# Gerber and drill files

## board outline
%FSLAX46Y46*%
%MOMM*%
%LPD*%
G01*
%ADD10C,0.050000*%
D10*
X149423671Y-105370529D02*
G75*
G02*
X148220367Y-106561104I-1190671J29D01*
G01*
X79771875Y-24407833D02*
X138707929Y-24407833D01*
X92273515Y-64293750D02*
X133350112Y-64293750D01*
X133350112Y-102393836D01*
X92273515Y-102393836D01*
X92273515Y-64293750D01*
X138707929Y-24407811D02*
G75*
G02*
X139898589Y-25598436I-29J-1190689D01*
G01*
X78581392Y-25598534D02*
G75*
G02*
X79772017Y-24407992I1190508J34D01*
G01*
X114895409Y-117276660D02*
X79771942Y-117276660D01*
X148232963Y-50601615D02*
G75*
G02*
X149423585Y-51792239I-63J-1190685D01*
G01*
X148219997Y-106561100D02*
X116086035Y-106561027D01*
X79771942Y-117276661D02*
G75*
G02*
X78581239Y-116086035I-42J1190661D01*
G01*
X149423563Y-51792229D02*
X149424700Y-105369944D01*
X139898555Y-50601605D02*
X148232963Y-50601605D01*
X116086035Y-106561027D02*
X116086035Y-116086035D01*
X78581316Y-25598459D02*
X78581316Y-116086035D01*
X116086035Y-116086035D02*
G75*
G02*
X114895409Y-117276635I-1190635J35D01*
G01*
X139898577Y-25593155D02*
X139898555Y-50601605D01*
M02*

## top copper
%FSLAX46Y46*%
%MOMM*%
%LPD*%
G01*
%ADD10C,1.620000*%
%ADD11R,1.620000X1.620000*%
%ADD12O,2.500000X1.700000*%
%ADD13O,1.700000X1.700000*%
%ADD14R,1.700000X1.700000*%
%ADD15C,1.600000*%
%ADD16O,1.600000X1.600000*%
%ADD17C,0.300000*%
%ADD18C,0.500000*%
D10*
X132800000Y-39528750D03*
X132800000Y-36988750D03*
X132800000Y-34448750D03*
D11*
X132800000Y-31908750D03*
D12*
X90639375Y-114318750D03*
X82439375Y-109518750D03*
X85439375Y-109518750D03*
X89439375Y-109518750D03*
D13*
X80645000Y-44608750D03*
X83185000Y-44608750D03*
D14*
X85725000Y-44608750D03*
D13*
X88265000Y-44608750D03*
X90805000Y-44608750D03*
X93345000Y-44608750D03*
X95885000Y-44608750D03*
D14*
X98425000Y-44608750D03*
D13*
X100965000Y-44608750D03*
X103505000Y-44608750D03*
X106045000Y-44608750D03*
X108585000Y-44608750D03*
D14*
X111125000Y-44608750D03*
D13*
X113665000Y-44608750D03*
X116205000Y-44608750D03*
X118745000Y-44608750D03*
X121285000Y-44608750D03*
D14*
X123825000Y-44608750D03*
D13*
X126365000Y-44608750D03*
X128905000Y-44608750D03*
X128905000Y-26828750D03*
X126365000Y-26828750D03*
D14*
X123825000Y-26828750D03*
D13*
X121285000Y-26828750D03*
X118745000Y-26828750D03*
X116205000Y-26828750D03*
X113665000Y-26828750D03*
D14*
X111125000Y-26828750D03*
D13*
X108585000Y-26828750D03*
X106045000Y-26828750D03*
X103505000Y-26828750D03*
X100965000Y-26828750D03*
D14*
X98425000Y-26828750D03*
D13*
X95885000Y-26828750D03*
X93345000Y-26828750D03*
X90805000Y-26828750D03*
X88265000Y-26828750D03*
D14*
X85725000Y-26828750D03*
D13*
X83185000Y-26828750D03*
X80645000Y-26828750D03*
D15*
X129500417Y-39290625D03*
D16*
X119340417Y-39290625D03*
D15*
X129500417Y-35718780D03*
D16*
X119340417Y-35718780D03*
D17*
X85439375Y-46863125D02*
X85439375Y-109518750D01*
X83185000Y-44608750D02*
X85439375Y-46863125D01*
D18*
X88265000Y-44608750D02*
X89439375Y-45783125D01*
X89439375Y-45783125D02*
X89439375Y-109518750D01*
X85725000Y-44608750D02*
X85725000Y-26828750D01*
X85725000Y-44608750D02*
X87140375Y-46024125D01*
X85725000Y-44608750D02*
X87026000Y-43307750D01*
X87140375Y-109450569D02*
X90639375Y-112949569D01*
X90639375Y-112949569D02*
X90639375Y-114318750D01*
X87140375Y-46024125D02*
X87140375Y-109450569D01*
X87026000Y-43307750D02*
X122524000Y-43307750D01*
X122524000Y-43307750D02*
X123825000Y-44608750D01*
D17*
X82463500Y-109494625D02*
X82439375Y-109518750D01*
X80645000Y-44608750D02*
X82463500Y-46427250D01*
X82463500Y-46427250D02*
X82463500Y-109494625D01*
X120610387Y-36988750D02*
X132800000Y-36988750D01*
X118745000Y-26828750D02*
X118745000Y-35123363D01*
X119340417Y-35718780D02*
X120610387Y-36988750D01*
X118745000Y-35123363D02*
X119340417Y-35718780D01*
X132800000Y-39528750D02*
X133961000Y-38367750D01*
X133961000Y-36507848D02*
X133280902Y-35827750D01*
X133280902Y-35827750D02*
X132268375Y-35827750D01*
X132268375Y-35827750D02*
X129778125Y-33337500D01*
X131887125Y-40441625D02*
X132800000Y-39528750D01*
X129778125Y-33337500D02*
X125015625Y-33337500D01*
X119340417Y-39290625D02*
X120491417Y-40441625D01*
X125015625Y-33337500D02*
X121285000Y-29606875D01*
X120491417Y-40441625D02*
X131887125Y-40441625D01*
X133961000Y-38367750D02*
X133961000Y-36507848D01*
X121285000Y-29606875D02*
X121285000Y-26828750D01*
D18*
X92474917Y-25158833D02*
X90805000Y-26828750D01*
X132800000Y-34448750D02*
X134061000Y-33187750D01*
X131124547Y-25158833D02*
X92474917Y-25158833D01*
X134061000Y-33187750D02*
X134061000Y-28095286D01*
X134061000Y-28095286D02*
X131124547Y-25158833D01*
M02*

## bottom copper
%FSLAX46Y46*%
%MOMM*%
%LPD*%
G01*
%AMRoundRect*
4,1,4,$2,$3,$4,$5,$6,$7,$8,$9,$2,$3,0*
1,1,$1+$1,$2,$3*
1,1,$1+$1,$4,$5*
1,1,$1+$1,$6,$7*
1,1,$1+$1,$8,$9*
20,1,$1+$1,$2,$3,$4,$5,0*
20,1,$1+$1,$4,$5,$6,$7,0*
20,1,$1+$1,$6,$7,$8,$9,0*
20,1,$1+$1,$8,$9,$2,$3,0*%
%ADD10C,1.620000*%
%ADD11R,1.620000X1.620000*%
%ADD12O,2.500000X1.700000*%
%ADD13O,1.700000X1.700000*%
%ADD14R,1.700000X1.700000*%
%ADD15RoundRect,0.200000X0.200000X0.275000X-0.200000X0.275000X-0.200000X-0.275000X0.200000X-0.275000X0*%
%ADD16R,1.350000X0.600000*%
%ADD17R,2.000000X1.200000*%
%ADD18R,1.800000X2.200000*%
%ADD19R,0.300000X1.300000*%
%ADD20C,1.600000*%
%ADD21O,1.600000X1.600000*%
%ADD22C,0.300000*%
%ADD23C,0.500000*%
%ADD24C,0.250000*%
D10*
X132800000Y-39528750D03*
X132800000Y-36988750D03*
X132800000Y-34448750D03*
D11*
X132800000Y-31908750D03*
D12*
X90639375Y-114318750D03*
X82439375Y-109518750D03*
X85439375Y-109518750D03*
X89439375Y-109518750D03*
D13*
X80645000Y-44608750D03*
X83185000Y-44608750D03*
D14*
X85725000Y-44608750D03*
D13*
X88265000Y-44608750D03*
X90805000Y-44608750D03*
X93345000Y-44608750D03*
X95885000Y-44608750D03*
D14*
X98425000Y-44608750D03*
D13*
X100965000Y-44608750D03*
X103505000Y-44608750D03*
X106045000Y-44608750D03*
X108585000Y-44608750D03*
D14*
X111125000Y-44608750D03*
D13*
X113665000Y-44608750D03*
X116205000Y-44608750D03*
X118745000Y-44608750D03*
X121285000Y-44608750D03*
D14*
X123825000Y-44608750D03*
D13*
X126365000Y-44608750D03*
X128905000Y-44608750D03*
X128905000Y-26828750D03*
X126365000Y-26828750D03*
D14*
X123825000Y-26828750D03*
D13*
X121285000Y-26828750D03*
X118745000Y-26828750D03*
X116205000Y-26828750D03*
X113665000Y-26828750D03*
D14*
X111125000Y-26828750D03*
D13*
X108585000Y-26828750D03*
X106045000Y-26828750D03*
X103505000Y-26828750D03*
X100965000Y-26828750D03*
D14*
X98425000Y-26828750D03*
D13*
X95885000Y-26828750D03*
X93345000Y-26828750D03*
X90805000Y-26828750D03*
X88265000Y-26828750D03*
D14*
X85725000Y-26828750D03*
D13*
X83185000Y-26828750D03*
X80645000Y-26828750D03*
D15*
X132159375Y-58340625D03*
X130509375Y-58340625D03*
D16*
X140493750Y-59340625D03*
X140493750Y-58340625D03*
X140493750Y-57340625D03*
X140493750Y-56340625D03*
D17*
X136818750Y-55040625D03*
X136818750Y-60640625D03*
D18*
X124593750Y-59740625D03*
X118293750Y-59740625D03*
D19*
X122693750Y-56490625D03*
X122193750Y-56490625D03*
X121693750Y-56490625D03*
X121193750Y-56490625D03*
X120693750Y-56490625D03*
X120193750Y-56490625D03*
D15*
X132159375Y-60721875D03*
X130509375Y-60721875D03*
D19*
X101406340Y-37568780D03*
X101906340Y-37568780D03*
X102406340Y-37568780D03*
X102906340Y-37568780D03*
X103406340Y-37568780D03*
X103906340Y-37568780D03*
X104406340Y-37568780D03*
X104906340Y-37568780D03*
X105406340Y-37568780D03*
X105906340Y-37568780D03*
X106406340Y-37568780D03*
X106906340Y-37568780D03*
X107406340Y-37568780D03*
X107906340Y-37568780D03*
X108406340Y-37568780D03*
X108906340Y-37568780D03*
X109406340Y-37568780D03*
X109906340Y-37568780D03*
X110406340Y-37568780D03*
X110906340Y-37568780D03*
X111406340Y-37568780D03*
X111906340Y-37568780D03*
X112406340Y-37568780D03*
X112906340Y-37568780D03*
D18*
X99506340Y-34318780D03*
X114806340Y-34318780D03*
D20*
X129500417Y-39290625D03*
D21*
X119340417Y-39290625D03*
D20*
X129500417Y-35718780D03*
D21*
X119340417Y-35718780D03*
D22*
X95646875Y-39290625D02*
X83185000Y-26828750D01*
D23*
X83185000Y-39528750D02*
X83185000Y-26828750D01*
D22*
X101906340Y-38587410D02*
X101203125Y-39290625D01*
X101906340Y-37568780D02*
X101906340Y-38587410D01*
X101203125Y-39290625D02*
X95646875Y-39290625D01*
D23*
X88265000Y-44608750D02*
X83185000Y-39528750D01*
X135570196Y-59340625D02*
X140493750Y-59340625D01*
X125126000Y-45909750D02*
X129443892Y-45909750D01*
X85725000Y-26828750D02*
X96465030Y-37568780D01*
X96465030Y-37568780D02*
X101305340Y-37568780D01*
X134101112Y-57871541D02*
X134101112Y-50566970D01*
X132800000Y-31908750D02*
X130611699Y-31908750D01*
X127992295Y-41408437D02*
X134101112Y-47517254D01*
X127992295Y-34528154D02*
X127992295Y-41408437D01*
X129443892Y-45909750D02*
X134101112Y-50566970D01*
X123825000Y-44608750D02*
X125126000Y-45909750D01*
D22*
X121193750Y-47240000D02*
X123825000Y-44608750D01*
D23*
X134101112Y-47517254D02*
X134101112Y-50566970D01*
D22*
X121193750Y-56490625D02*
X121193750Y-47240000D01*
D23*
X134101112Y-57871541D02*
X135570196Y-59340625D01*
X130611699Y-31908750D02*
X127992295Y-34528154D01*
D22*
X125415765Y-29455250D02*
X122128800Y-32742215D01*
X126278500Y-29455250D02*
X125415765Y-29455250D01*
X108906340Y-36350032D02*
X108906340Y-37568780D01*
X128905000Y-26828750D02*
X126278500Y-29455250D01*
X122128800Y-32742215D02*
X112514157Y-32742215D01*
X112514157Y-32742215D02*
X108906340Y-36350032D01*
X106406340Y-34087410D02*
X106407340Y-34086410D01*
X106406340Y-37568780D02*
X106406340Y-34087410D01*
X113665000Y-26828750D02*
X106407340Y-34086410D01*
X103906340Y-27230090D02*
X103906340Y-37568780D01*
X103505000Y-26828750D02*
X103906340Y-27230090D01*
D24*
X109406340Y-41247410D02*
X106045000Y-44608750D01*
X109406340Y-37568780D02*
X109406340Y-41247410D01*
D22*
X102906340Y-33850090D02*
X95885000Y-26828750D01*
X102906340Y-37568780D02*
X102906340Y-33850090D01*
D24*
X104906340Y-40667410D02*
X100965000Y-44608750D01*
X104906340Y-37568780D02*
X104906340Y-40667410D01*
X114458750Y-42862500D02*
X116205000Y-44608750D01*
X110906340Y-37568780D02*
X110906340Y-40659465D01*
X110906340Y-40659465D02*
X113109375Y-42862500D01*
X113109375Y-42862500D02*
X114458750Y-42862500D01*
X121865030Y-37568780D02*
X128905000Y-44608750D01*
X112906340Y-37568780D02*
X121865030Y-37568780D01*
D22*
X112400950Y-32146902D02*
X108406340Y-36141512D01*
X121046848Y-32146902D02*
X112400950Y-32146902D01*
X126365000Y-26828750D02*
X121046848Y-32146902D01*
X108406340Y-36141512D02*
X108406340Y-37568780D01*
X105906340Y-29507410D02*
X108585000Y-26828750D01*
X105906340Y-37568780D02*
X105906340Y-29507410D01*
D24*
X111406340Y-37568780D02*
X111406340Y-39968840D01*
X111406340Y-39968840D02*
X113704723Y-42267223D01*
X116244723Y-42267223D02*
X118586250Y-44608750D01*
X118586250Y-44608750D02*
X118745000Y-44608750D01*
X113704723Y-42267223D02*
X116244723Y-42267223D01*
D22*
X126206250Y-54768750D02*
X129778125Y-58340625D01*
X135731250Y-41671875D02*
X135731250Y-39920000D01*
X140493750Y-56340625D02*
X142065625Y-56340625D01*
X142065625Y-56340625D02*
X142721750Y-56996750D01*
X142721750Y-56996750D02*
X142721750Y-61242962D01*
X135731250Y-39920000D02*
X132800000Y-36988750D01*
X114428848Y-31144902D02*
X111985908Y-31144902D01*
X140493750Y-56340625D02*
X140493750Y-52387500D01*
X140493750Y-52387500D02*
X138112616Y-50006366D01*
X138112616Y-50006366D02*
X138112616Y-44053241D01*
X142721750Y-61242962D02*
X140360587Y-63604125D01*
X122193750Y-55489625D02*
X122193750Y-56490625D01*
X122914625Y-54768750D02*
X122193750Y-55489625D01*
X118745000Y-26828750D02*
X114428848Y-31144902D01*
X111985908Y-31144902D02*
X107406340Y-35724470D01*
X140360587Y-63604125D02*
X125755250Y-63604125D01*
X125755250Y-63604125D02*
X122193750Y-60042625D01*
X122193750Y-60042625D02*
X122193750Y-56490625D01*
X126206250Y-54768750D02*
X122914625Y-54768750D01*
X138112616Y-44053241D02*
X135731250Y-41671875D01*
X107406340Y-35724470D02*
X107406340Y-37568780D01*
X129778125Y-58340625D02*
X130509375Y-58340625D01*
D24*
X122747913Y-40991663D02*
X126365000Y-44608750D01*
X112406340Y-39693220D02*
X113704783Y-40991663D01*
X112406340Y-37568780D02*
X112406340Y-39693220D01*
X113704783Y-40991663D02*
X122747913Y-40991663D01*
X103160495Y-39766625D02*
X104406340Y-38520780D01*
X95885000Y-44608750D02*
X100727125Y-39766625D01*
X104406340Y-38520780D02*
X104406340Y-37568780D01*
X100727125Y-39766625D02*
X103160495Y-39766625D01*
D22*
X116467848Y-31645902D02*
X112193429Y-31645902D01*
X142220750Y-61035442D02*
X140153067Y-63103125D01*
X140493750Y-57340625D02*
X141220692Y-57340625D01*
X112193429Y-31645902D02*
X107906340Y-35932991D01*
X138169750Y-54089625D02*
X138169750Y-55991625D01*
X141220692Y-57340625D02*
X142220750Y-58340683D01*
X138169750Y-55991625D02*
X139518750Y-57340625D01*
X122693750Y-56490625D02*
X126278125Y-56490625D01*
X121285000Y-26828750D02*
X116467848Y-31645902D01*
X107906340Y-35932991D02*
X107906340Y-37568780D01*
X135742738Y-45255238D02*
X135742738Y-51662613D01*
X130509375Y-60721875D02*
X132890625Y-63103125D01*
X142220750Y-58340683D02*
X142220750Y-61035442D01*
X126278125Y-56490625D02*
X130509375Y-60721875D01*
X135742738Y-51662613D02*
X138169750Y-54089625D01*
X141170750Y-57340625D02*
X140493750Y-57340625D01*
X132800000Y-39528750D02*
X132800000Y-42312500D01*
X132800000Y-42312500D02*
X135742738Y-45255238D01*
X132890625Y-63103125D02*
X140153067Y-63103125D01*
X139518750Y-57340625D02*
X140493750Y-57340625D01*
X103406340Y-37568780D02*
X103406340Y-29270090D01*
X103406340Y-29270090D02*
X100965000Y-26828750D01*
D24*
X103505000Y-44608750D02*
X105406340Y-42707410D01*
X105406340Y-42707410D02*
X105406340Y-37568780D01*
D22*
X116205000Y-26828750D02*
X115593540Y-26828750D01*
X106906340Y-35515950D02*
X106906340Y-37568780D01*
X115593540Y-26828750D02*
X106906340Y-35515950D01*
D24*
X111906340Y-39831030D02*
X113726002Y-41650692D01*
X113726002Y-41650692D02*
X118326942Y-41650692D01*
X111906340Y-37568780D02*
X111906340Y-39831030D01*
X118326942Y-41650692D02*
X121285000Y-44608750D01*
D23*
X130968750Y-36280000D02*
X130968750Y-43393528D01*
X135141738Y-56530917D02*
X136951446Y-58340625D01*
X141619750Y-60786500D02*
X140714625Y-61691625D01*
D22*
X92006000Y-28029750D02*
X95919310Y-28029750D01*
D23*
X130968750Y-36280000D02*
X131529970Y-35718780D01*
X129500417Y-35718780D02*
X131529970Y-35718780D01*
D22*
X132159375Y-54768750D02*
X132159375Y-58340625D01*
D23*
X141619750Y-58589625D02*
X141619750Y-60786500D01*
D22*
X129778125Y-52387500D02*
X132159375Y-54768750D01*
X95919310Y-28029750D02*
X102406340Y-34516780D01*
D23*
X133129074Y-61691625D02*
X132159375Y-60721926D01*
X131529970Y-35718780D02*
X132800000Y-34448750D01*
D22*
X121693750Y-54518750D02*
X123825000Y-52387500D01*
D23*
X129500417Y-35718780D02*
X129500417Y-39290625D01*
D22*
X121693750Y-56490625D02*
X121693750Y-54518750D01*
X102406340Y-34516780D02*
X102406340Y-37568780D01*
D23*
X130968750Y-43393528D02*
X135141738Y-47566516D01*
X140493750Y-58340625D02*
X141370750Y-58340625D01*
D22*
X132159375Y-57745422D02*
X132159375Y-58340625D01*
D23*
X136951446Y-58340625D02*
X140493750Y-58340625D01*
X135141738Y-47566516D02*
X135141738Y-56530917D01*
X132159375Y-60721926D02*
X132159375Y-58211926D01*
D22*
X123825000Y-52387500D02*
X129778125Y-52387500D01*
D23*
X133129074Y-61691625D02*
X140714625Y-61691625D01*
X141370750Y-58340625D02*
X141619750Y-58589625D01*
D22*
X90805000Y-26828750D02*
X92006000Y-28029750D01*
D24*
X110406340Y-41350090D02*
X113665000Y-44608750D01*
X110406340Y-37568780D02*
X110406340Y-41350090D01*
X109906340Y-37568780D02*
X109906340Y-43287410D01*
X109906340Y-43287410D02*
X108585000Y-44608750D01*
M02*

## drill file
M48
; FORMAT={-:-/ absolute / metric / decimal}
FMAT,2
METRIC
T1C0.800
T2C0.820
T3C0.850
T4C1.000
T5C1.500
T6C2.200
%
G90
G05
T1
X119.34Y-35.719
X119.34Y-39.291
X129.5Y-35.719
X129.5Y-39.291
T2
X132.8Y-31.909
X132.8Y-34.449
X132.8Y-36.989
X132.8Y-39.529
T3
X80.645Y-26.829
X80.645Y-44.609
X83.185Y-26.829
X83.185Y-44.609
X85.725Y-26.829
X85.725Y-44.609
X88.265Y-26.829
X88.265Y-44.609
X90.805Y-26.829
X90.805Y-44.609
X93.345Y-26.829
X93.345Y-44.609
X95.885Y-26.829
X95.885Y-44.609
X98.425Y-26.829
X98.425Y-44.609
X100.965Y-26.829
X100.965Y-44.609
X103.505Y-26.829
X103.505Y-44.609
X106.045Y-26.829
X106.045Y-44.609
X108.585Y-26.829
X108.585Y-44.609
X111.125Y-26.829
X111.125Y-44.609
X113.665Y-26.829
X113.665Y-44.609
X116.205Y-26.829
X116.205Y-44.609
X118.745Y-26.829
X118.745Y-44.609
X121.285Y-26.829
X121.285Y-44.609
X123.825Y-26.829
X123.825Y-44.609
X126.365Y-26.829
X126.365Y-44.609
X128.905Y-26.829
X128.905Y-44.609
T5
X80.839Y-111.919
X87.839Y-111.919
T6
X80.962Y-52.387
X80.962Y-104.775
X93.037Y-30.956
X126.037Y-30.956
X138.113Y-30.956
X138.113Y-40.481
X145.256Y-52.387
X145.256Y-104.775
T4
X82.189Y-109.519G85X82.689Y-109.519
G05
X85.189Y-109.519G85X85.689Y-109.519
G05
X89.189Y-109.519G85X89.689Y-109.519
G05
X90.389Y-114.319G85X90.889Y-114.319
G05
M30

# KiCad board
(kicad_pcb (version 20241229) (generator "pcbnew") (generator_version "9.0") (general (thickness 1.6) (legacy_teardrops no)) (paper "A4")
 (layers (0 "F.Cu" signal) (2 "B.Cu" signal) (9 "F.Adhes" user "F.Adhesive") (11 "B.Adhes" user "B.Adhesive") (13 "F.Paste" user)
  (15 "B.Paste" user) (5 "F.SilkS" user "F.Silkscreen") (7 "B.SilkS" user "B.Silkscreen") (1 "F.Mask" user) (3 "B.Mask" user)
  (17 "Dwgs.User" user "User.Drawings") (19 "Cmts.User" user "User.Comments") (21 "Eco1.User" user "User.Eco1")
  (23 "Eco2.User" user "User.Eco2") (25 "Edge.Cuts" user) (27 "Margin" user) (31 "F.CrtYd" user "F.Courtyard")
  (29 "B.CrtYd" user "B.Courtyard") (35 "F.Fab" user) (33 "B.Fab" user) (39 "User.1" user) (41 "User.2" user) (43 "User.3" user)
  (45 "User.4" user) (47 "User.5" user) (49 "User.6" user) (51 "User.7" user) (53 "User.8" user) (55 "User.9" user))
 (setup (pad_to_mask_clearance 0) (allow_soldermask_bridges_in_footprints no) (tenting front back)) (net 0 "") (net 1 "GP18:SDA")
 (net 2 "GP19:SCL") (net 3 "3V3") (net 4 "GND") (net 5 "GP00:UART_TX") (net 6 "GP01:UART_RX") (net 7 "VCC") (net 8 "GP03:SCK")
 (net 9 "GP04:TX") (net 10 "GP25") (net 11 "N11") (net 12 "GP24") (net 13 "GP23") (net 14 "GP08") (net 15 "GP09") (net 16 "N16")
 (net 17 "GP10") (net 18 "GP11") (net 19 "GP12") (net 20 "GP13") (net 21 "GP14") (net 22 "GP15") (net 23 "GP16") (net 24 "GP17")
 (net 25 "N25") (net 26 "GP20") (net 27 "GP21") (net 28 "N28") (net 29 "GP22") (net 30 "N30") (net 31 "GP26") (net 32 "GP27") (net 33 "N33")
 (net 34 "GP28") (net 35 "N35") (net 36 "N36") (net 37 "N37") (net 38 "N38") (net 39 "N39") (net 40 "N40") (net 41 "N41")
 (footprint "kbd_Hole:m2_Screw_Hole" (layer "F.Cu") (at 145.25625 52.3875)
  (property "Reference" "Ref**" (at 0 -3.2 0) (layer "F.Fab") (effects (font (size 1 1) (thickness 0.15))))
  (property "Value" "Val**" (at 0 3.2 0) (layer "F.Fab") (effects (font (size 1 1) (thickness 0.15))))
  (pad "" np_thru_hole circle (at 0 0) (size 2.2 2.2) (drill 2.2) (layers "*.Cu" "*.Mask")))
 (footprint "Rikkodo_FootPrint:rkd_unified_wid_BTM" (layer "F.Cu") (at 109.5375 30.95625)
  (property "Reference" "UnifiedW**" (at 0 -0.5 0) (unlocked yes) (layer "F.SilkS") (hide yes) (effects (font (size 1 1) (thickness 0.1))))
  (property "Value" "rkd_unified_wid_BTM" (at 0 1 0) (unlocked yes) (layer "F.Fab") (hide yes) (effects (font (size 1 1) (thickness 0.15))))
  (pad "" np_thru_hole circle (at -16.5 0) (size 2.2 2.2) (drill 2.2) (layers "*.Cu" "*.Mask"))
  (pad "" np_thru_hole circle (at 16.5 0) (size 2.2 2.2) (drill 2.2) (layers "*.Cu" "*.Mask")))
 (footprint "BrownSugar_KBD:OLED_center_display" (layer "F.Cu") (at 114.3 35.71875 90)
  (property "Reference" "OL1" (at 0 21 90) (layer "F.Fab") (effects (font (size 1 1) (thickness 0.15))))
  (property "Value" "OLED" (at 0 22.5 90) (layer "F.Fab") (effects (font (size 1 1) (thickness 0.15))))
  (pad "1" thru_hole circle (at -3.81 18.5 90) (size 1.62 1.62) (drill 0.82) (layers "*.Cu" "*.Mask") (remove_unused_layers no)
   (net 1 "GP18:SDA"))
  (pad "2" thru_hole circle (at -1.27 18.5 90) (size 1.62 1.62) (drill 0.82) (layers "*.Cu" "*.Mask") (remove_unused_layers no)
   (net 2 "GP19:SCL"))
  (pad "3" thru_hole circle (at 1.27 18.5 90) (size 1.62 1.62) (drill 0.82) (layers "*.Cu" "*.Mask") (remove_unused_layers no) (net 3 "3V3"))
  (pad "4" thru_hole rect (at 3.81 18.5 90) (size 1.62 1.62) (drill 0.82) (layers "*.Cu" "*.Mask") (remove_unused_layers no) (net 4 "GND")))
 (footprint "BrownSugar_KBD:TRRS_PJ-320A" (layer "F.Cu") (at 79.239375 111.91875 90)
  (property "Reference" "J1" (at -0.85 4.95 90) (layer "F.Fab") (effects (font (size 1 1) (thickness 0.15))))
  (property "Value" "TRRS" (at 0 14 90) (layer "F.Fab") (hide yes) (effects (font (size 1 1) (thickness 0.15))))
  (pad "" np_thru_hole circle (at 0 1.6 90) (size 1.5 1.5) (drill 1.5) (layers "*.Cu" "*.Mask"))
  (pad "" np_thru_hole circle (at 0 8.6 90) (size 1.5 1.5) (drill 1.5) (layers "*.Cu" "*.Mask"))
  (pad "A" thru_hole oval (at -2.4 11.4 90) (size 1.7 2.5) (drill oval 1 1.5) (layers "*.Cu" "*.Mask") (remove_unused_layers no)
   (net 4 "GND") (clearance 0.15))
  (pad "B" thru_hole oval (at 2.4 3.2 90) (size 1.7 2.5) (drill oval 1 1.5) (layers "*.Cu" "*.Mask") (remove_unused_layers no)
   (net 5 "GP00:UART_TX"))
  (pad "C" thru_hole oval (at 2.4 6.2 90) (size 1.7 2.5) (drill oval 1 1.5) (layers "*.Cu" "*.Mask") (remove_unused_layers no)
   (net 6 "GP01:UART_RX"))
  (pad "D" thru_hole oval (at 2.4 10.2 90) (size 1.7 2.5) (drill oval 1 1.5) (layers "*.Cu" "*.Mask") (remove_unused_layers no)
   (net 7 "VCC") (clearance 0.15)))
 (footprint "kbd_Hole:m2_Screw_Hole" (layer "F.Cu") (at 80.9625 52.3875)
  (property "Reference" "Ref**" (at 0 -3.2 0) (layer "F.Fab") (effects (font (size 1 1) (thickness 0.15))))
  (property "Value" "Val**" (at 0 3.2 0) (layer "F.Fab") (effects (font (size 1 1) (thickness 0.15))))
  (pad "" np_thru_hole circle (at 0 0) (size 2.2 2.2) (drill 2.2) (layers "*.Cu" "*.Mask")))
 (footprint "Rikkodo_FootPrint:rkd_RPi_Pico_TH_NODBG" (layer "F.Cu") (at 104.775 35.71875 90)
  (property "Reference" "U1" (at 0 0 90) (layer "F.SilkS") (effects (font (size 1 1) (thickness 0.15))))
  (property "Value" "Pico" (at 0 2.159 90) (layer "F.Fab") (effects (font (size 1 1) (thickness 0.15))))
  (pad "1" thru_hole oval (at -8.89 -24.13 90) (size 1.7 1.7) (drill 0.85) (layers "*.Cu" "*.Mask") (remove_unused_layers no)
   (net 5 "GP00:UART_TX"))
  (pad "2" thru_hole oval (at -8.89 -21.59 90) (size 1.7 1.7) (drill 0.85) (layers "*.Cu" "*.Mask") (remove_unused_layers no)
   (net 6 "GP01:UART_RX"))
  (pad "3" thru_hole rect (at -8.89 -19.05 90) (size 1.7 1.7) (drill 0.85) (layers "*.Cu" "*.Mask") (remove_unused_layers no) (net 4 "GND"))
  (pad "4" thru_hole oval (at -8.89 -16.51 90) (size 1.7 1.7) (drill 0.85) (layers "*.Cu" "*.Mask") (remove_unused_layers no) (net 7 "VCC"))
  (pad "5" thru_hole oval (at -8.89 -13.97 90) (size 1.7 1.7) (drill 0.85) (layers "*.Cu" "*.Mask") (remove_unused_layers no)
   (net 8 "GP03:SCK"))
  (pad "6" thru_hole oval (at -8.89 -11.43 90) (size 1.7 1.7) (drill 0.85) (layers "*.Cu" "*.Mask") (remove_unused_layers no)
   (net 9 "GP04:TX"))
  (pad "7" thru_hole oval (at -8.89 -8.89 90) (size 1.7 1.7) (drill 0.85) (layers "*.Cu" "*.Mask") (remove_unused_layers no) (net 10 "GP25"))
  (pad "8" thru_hole rect (at -8.89 -6.35 90) (size 1.7 1.7) (drill 0.85) (layers "*.Cu" "*.Mask") (remove_unused_layers no) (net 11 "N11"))
  (pad "9" thru_hole oval (at -8.89 -3.81 90) (size 1.7 1.7) (drill 0.85) (layers "*.Cu" "*.Mask") (remove_unused_layers no) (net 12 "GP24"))
  (pad "10" thru_hole oval (at -8.89 -1.27 90) (size 1.7 1.7) (drill 0.85) (layers "*.Cu" "*.Mask") (remove_unused_layers no)
   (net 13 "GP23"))
  (pad "11" thru_hole oval (at -8.89 1.27 90) (size 1.7 1.7) (drill 0.85) (layers "*.Cu" "*.Mask") (remove_unused_layers no) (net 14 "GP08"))
  (pad "12" thru_hole oval (at -8.89 3.81 90) (size 1.7 1.7) (drill 0.85) (layers "*.Cu" "*.Mask") (remove_unused_layers no) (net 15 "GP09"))
  (pad "13" thru_hole rect (at -8.89 6.35 90) (size 1.7 1.7) (drill 0.85) (layers "*.Cu" "*.Mask") (remove_unused_layers no) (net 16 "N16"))
  (pad "14" thru_hole oval (at -8.89 8.89 90) (size 1.7 1.7) (drill 0.85) (layers "*.Cu" "*.Mask") (remove_unused_layers no) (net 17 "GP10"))
  (pad "15" thru_hole oval (at -8.89 11.43 90) (size 1.7 1.7) (drill 0.85) (layers "*.Cu" "*.Mask") (remove_unused_layers no)
   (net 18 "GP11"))
  (pad "16" thru_hole oval (at -8.89 13.97 90) (size 1.7 1.7) (drill 0.85) (layers "*.Cu" "*.Mask") (remove_unused_layers no)
   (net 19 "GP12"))
  (pad "17" thru_hole oval (at -8.89 16.51 90) (size 1.7 1.7) (drill 0.85) (layers "*.Cu" "*.Mask") (remove_unused_layers no)
   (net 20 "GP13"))
  (pad "18" thru_hole rect (at -8.89 19.05 90) (size 1.7 1.7) (drill 0.85) (layers "*.Cu" "*.Mask") (remove_unused_layers no) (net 4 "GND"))
  (pad "19" thru_hole oval (at -8.89 21.59 90) (size 1.7 1.7) (drill 0.85) (layers "*.Cu" "*.Mask") (remove_unused_layers no)
   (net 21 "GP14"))
  (pad "20" thru_hole oval (at -8.89 24.13 90) (size 1.7 1.7) (drill 0.85) (layers "*.Cu" "*.Mask") (remove_unused_layers no)
   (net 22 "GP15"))
  (pad "21" thru_hole oval (at 8.89 24.13 90) (size 1.7 1.7) (drill 0.85) (layers "*.Cu" "*.Mask") (remove_unused_layers no) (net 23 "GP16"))
  (pad "22" thru_hole oval (at 8.89 21.59 90) (size 1.7 1.7) (drill 0.85) (layers "*.Cu" "*.Mask") (remove_unused_layers no) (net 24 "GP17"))
  (pad "23" thru_hole rect (at 8.89 19.05 90) (size 1.7 1.7) (drill 0.85) (layers "*.Cu" "*.Mask") (remove_unused_layers no) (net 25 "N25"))
  (pad "24" thru_hole oval (at 8.89 16.51 90) (size 1.7 1.7) (drill 0.85) (layers "*.Cu" "*.Mask") (remove_unused_layers no)
   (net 1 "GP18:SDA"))
  (pad "25" thru_hole oval (at 8.89 13.97 90) (size 1.7 1.7) (drill 0.85) (layers "*.Cu" "*.Mask") (remove_unused_layers no)
   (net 2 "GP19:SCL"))
  (pad "26" thru_hole oval (at 8.89 11.43 90) (size 1.7 1.7) (drill 0.85) (layers "*.Cu" "*.Mask") (remove_unused_layers no) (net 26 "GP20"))
  (pad "27" thru_hole oval (at 8.89 8.89 90) (size 1.7 1.7) (drill 0.85) (layers "*.Cu" "*.Mask") (remove_unused_layers no) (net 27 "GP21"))
  (pad "28" thru_hole rect (at 8.89 6.35 90) (size 1.7 1.7) (drill 0.85) (layers "*.Cu" "*.Mask") (remove_unused_layers no) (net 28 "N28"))
  (pad "29" thru_hole oval (at 8.89 3.81 90) (size 1.7 1.7) (drill 0.85) (layers "*.Cu" "*.Mask") (remove_unused_layers no) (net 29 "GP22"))
  (pad "30" thru_hole oval (at 8.89 1.27 90) (size 1.7 1.7) (drill 0.85) (layers "*.Cu" "*.Mask") (remove_unused_layers no) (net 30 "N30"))
  (pad "31" thru_hole oval (at 8.89 -1.27 90) (size 1.7 1.7) (drill 0.85) (layers "*.Cu" "*.Mask") (remove_unused_layers no) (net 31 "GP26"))
  (pad "32" thru_hole oval (at 8.89 -3.81 90) (size 1.7 1.7) (drill 0.85) (layers "*.Cu" "*.Mask") (remove_unused_layers no) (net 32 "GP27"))
  (pad "33" thru_hole rect (at 8.89 -6.35 90) (size 1.7 1.7) (drill 0.85) (layers "*.Cu" "*.Mask") (remove_unused_layers no) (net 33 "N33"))
  (pad "34" thru_hole oval (at 8.89 -8.89 90) (size 1.7 1.7) (drill 0.85) (layers "*.Cu" "*.Mask") (remove_unused_layers no) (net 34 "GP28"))
  (pad "35" thru_hole oval (at 8.89 -11.43 90) (size 1.7 1.7) (drill 0.85) (layers "*.Cu" "*.Mask") (remove_unused_layers no) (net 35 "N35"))
  (pad "36" thru_hole oval (at 8.89 -13.97 90) (size 1.7 1.7) (drill 0.85) (layers "*.Cu" "*.Mask") (remove_unused_layers no) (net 3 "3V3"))
  (pad "37" thru_hole oval (at 8.89 -16.51 90) (size 1.7 1.7) (drill 0.85) (layers "*.Cu" "*.Mask") (remove_unused_layers no) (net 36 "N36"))
  (pad "38" thru_hole rect (at 8.89 -19.05 90) (size 1.7 1.7) (drill 0.85) (layers "*.Cu" "*.Mask") (remove_unused_layers no) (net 4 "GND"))
  (pad "39" thru_hole oval (at 8.89 -21.59 90) (size 1.7 1.7) (drill 0.85) (layers "*.Cu" "*.Mask") (remove_unused_layers no) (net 7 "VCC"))
  (pad "40" thru_hole oval (at 8.89 -24.13 90) (size 1.7 1.7) (drill 0.85) (layers "*.Cu" "*.Mask") (remove_unused_layers no) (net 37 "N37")))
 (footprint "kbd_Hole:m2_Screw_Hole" (layer "F.Cu") (at 145.25625 104.775)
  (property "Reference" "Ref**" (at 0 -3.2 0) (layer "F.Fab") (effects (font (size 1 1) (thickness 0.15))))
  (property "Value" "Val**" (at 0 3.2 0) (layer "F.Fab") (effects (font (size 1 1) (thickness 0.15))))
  (pad "" np_thru_hole circle (at 0 0) (size 2.2 2.2) (drill 2.2) (layers "*.Cu" "*.Mask")))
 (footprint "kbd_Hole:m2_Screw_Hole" (layer "F.Cu") (at 80.9625 104.775)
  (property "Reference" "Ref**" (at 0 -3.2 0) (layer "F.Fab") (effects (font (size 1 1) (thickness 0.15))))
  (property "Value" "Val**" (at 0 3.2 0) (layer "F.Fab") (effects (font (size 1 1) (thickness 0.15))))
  (pad "" np_thru_hole circle (at 0 0) (size 2.2 2.2) (drill 2.2) (layers "*.Cu" "*.Mask")))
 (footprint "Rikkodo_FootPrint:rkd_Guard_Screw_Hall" (layer "F.Cu") (at 108.346966 35.71878)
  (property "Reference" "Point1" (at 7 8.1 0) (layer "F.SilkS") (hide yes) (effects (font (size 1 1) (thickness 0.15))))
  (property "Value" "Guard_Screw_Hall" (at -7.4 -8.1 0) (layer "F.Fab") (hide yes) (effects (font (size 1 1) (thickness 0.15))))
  (pad "" np_thru_hole circle (at 29.765625 -4.7625) (size 2.2 2.2) (drill 2.2) (layers "*.Cu" "*.Mask"))
  (pad "" np_thru_hole circle (at 29.765625 4.7625) (size 2.2 2.2) (drill 2.2) (layers "*.Cu" "*.Mask")))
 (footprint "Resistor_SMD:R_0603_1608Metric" (layer "B.Cu") (at 131.334375 58.340625 180)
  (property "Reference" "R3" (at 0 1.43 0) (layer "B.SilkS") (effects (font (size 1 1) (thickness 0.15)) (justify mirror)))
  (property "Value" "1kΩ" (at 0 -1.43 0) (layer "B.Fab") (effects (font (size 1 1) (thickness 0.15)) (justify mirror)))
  (pad "1" smd roundrect (at -0.825 0 180) (size 0.8 0.95) (layers "B.Cu" "B.Mask" "B.Paste") (roundrect_rratio 0.25) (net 3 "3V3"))
  (pad "2" smd roundrect (at 0.825 0 180) (size 0.8 0.95) (layers "B.Cu" "B.Mask" "B.Paste") (roundrect_rratio 0.25) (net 2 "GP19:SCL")))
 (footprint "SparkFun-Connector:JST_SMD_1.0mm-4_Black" (layer "B.Cu") (at 140.49375 57.840625 90)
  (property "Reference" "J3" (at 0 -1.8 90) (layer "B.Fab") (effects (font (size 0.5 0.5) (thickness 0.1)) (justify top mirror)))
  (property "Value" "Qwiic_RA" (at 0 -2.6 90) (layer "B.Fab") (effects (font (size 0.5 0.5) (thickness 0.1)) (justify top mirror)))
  (pad "1" smd rect (at -1.5 0 90) (size 0.6 1.35) (layers "B.Cu" "B.Mask" "B.Paste") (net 4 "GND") (thermal_bridge_angle 0))
  (pad "2" smd rect (at -0.5 0 90) (size 0.6 1.35) (layers "B.Cu" "B.Mask" "B.Paste") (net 3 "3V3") (thermal_bridge_angle 0))
  (pad "3" smd rect (at 0.5 0 90) (size 0.6 1.35) (layers "B.Cu" "B.Mask" "B.Paste") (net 1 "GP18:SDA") (thermal_bridge_angle 0))
  (pad "4" smd rect (at 1.5 0 90) (size 0.6 1.35) (layers "B.Cu" "B.Mask" "B.Paste") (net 2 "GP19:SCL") (thermal_bridge_angle 0))
  (pad "NC1" smd rect (at 2.8 -3.675 90) (size 1.2 2) (layers "B.Cu" "B.Mask" "B.Paste") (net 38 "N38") (thermal_bridge_angle 0))
  (pad "NC2" smd rect (at -2.8 -3.675 90) (size 1.2 2) (layers "B.Cu" "B.Mask" "B.Paste") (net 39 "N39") (thermal_bridge_angle 0)))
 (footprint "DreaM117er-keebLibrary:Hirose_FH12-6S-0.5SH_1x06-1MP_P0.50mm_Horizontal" (layer "B.Cu") (at 121.44375 58.340625 180)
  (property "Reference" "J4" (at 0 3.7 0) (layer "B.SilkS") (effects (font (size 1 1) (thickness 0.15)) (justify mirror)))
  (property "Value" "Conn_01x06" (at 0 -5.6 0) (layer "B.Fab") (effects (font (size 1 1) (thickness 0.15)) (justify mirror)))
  (pad "" smd rect (at -3.15 -1.4 180) (size 1.8 2.2) (layers "B.Cu" "B.Mask" "B.Paste"))
  (pad "" smd rect (at 3.15 -1.4 180) (size 1.8 2.2) (layers "B.Cu" "B.Mask" "B.Paste"))
  (pad "1" smd rect (at -1.25 1.85 180) (size 0.3 1.3) (layers "B.Cu" "B.Mask" "B.Paste") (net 1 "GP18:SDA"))
  (pad "2" smd rect (at -0.75 1.85 180) (size 0.3 1.3) (layers "B.Cu" "B.Mask" "B.Paste") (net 2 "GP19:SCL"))
  (pad "3" smd rect (at -0.25 1.85 180) (size 0.3 1.3) (layers "B.Cu" "B.Mask" "B.Paste") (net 3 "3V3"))
  (pad "4" smd rect (at 0.25 1.85 180) (size 0.3 1.3) (layers "B.Cu" "B.Mask" "B.Paste") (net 4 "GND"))
  (pad "5" smd rect (at 0.75 1.85 180) (size 0.3 1.3) (layers "B.Cu" "B.Mask" "B.Paste") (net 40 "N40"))
  (pad "6" smd rect (at 1.25 1.85 180) (size 0.3 1.3) (layers "B.Cu" "B.Mask" "B.Paste") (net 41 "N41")))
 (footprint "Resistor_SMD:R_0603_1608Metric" (layer "B.Cu") (at 131.334375 60.721875 180)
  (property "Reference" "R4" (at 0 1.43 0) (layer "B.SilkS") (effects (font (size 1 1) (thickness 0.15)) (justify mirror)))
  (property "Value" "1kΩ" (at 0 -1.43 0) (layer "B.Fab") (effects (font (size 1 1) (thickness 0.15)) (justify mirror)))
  (pad "1" smd roundrect (at -0.825 0 180) (size 0.8 0.95) (layers "B.Cu" "B.Mask" "B.Paste") (roundrect_rratio 0.25) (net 3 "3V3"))
  (pad "2" smd roundrect (at 0.825 0 180) (size 0.8 0.95) (layers "B.Cu" "B.Mask" "B.Paste") (roundrect_rratio 0.25) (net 1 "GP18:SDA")))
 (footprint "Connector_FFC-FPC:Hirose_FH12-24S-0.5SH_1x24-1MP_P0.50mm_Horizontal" (layer "B.Cu") (at 107.15634 35.71878)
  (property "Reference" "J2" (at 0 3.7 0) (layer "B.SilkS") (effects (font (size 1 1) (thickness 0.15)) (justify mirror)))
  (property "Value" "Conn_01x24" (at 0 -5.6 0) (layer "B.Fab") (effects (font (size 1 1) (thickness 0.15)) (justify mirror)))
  (pad "1" smd rect (at -5.75 1.85) (size 0.3 1.3) (layers "B.Cu" "B.Mask" "B.Paste") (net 4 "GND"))
  (pad "2" smd rect (at -5.25 1.85) (size 0.3 1.3) (layers "B.Cu" "B.Mask" "B.Paste") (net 7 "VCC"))
  (pad "3" smd rect (at -4.75 1.85) (size 0.3 1.3) (layers "B.Cu" "B.Mask" "B.Paste") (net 3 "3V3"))
  (pad "4" smd rect (at -4.25 1.85) (size 0.3 1.3) (layers "B.Cu" "B.Mask" "B.Paste") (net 34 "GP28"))
  (pad "5" smd rect (at -3.75 1.85) (size 0.3 1.3) (layers "B.Cu" "B.Mask" "B.Paste") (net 32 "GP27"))
  (pad "6" smd rect (at -3.25 1.85) (size 0.3 1.3) (layers "B.Cu" "B.Mask" "B.Paste") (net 31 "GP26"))
  (pad "7" smd rect (at -2.75 1.85) (size 0.3 1.3) (layers "B.Cu" "B.Mask" "B.Paste") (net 10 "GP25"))
  (pad "8" smd rect (at -2.25 1.85) (size 0.3 1.3) (layers "B.Cu" "B.Mask" "B.Paste") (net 12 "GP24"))
  (pad "9" smd rect (at -1.75 1.85) (size 0.3 1.3) (layers "B.Cu" "B.Mask" "B.Paste") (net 13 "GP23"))
  (pad "10" smd rect (at -1.25 1.85) (size 0.3 1.3) (layers "B.Cu" "B.Mask" "B.Paste") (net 29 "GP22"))
  (pad "11" smd rect (at -0.75 1.85) (size 0.3 1.3) (layers "B.Cu" "B.Mask" "B.Paste") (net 27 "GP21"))
  (pad "12" smd rect (at -0.25 1.85) (size 0.3 1.3) (layers "B.Cu" "B.Mask" "B.Paste") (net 26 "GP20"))
  (pad "13" smd rect (at 0.25 1.85) (size 0.3 1.3) (layers "B.Cu" "B.Mask" "B.Paste") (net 2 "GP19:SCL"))
  (pad "14" smd rect (at 0.75 1.85) (size 0.3 1.3) (layers "B.Cu" "B.Mask" "B.Paste") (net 1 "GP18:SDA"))
  (pad "15" smd rect (at 1.25 1.85) (size 0.3 1.3) (layers "B.Cu" "B.Mask" "B.Paste") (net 24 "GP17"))
  (pad "16" smd rect (at 1.75 1.85) (size 0.3 1.3) (layers "B.Cu" "B.Mask" "B.Paste") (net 23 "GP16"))
  (pad "17" smd rect (at 2.25 1.85) (size 0.3 1.3) (layers "B.Cu" "B.Mask" "B.Paste") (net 14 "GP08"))
  (pad "18" smd rect (at 2.75 1.85) (size 0.3 1.3) (layers "B.Cu" "B.Mask" "B.Paste") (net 15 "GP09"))
  (pad "19" smd rect (at 3.25 1.85) (size 0.3 1.3) (layers "B.Cu" "B.Mask" "B.Paste") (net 17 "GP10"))
  (pad "20" smd rect (at 3.75 1.85) (size 0.3 1.3) (layers "B.Cu" "B.Mask" "B.Paste") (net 18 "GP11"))
  (pad "21" smd rect (at 4.25 1.85) (size 0.3 1.3) (layers "B.Cu" "B.Mask" "B.Paste") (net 19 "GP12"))
  (pad "22" smd rect (at 4.75 1.85) (size 0.3 1.3) (layers "B.Cu" "B.Mask" "B.Paste") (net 20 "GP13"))
  (pad "23" smd rect (at 5.25 1.85) (size 0.3 1.3) (layers "B.Cu" "B.Mask" "B.Paste") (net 21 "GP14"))
  (pad "24" smd rect (at 5.75 1.85) (size 0.3 1.3) (layers "B.Cu" "B.Mask" "B.Paste") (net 22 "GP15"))
  (pad "MP" smd rect (at -7.65 -1.4) (size 1.8 2.2) (layers "B.Cu" "B.Mask" "B.Paste"))
  (pad "MP" smd rect (at 7.65 -1.4) (size 1.8 2.2) (layers "B.Cu" "B.Mask" "B.Paste")))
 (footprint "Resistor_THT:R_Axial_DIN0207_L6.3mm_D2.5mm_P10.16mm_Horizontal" (layer "B.Cu") (at 129.500417 39.290625 180)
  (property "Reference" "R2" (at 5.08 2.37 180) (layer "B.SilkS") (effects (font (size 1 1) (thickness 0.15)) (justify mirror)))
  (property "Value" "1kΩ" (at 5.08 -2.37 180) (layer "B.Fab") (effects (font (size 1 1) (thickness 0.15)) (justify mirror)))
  (pad "1" thru_hole circle (at 0 0 180) (size 1.6 1.6) (drill 0.8) (layers "*.Cu" "*.Mask") (remove_unused_layers no) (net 3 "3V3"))
  (pad "2" thru_hole oval (at 10.16 0 180) (size 1.6 1.6) (drill 0.8) (layers "*.Cu" "*.Mask") (remove_unused_layers no) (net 1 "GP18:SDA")))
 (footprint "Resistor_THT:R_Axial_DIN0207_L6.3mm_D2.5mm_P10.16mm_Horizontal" (layer "B.Cu") (at 129.500417 35.71878 180)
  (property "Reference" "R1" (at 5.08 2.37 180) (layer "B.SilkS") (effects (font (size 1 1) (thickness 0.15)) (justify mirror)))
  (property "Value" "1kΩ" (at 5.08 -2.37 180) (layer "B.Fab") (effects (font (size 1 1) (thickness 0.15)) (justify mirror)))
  (pad "1" thru_hole circle (at 0 0 180) (size 1.6 1.6) (drill 0.8) (layers "*.Cu" "*.Mask") (remove_unused_layers no) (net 3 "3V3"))
  (pad "2" thru_hole oval (at 10.16 0 180) (size 1.6 1.6) (drill 0.8) (layers "*.Cu" "*.Mask") (remove_unused_layers no) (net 2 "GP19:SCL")))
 (gr_arc (start 149.423671 105.370529) (mid 149.070452 106.216908) (end 148.220367 106.561112) (stroke (width 0.05) (type default))
  (layer "Edge.Cuts"))
 (gr_line (start 79.771875 24.407833) (end 138.707929 24.407833) (stroke (width 0.05) (type default)) (layer "Edge.Cuts"))
 (gr_rect (start 92.273515 64.29375) (end 133.350112 102.393836) (stroke (width 0.05) (type default)) (fill no) (layer "Edge.Cuts"))
 (gr_arc (start 138.707929 24.407811) (mid 139.549836 24.756536) (end 139.898577 25.598436) (stroke (width 0.05) (type default))
  (layer "Edge.Cuts"))
 (gr_arc (start 78.581392 25.598534) (mid 78.930096 24.756613) (end 79.772017 24.407909) (stroke (width 0.05) (type default))
  (layer "Edge.Cuts"))
 (gr_line (start 114.895409 117.27666) (end 79.771942 117.27666) (stroke (width 0.05) (type default)) (layer "Edge.Cuts"))
 (gr_arc (start 148.232963 50.601615) (mid 149.074854 50.950348) (end 149.423587 51.792239) (stroke (width 0.05) (type default))
  (layer "Edge.Cuts"))
 (gr_line (start 148.219997 106.5611) (end 116.086035 106.561027) (stroke (width 0.05) (type default)) (layer "Edge.Cuts"))
 (gr_arc (start 79.771942 117.276661) (mid 78.930042 116.927935) (end 78.581316 116.086035) (stroke (width 0.05) (type default))
  (layer "Edge.Cuts"))
 (gr_line (start 149.423563 51.792229) (end 149.4247 105.369944) (stroke (width 0.05) (type default)) (layer "Edge.Cuts"))
 (gr_line (start 139.898555 50.601605) (end 148.232963 50.601605) (stroke (width 0.05) (type default)) (layer "Edge.Cuts"))
 (gr_line (start 116.086035 106.561027) (end 116.086035 116.086035) (stroke (width 0.05) (type default)) (layer "Edge.Cuts"))
 (gr_line (start 78.581316 25.598459) (end 78.581316 116.086035) (stroke (width 0.05) (type default)) (layer "Edge.Cuts"))
 (gr_arc (start 116.086035 116.086035) (mid 115.737309 116.927935) (end 114.895409 117.276661) (stroke (width 0.05) (type default))
  (layer "Edge.Cuts"))
 (gr_line (start 139.898577 25.593155) (end 139.898555 50.601605) (stroke (width 0.05) (type default)) (layer "Edge.Cuts"))
 (segment (start 85.439375 46.863125) (end 85.439375 109.51875) (width 0.3) (layer "F.Cu") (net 6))
 (segment (start 83.185 44.60875) (end 85.439375 46.863125) (width 0.3) (layer "F.Cu") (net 6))
 (segment (start 88.265 44.60875) (end 89.439375 45.783125) (width 0.5) (layer "F.Cu") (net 7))
 (segment (start 89.439375 45.783125) (end 89.439375 109.51875) (width 0.5) (layer "F.Cu") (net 7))
 (segment (start 95.646875 39.290625) (end 83.185 26.82875) (width 0.3) (layer "B.Cu") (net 7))
 (segment (start 83.185 39.52875) (end 83.185 26.82875) (width 0.5) (layer "B.Cu") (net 7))
 (segment (start 101.90634 38.58741) (end 101.203125 39.290625) (width 0.3) (layer "B.Cu") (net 7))
 (segment (start 101.90634 37.56878) (end 101.90634 38.58741) (width 0.3) (layer "B.Cu") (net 7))
 (segment (start 101.203125 39.290625) (end 95.646875 39.290625) (width 0.3) (layer "B.Cu") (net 7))
 (segment (start 88.265 44.60875) (end 83.185 39.52875) (width 0.5) (layer "B.Cu") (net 7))
 (segment (start 85.725 44.60875) (end 85.725 26.82875) (width 0.5) (layer "F.Cu") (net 4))
 (segment (start 85.725 44.60875) (end 87.140375 46.024125) (width 0.5) (layer "F.Cu") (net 4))
 (segment (start 85.725 44.60875) (end 87.026 43.30775) (width 0.5) (layer "F.Cu") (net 4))
 (segment (start 87.140375 109.450569) (end 90.639375 112.949569) (width 0.5) (layer "F.Cu") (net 4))
 (segment (start 90.639375 112.949569) (end 90.639375 114.31875) (width 0.5) (layer "F.Cu") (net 4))
 (segment (start 87.140375 46.024125) (end 87.140375 109.450569) (width 0.5) (layer "F.Cu") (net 4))
 (segment (start 87.026 43.30775) (end 122.524 43.30775) (width 0.5) (layer "F.Cu") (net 4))
 (segment (start 122.524 43.30775) (end 123.825 44.60875) (width 0.5) (layer "F.Cu") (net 4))
 (segment (start 135.570196 59.340625) (end 140.49375 59.340625) (width 0.5) (layer "B.Cu") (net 4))
 (segment (start 125.126 45.90975) (end 129.443892 45.90975) (width 0.5) (layer "B.Cu") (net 4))
 (segment (start 85.725 26.82875) (end 96.46503 37.56878) (width 0.5) (layer "B.Cu") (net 4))
 (segment (start 96.46503 37.56878) (end 101.30534 37.56878) (width 0.5) (layer "B.Cu") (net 4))
 (segment (start 134.101112 57.871541) (end 134.101112 50.56697) (width 0.5) (layer "B.Cu") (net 4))
 (segment (start 132.8 31.90875) (end 130.611699 31.90875) (width 0.5) (layer "B.Cu") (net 4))
 (segment (start 127.992295 41.408437) (end 134.101112 47.517254) (width 0.5) (layer "B.Cu") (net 4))
 (segment (start 127.992295 34.528154) (end 127.992295 41.408437) (width 0.5) (layer "B.Cu") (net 4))
 (segment (start 129.443892 45.90975) (end 134.101112 50.56697) (width 0.5) (layer "B.Cu") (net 4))
 (segment (start 123.825 44.60875) (end 125.126 45.90975) (width 0.5) (layer "B.Cu") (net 4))
 (segment (start 121.19375 47.24) (end 123.825 44.60875) (width 0.3) (layer "B.Cu") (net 4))
 (segment (start 134.101112 47.517254) (end 134.101112 50.56697) (width 0.5) (layer "B.Cu") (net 4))
 (segment (start 121.19375 56.490625) (end 121.19375 47.24) (width 0.3) (layer "B.Cu") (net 4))
 (segment (start 134.101112 57.871541) (end 135.570196 59.340625) (width 0.5) (layer "B.Cu") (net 4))
 (segment (start 130.611699 31.90875) (end 127.992295 34.528154) (width 0.5) (layer "B.Cu") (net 4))
 (segment (start 82.4635 109.494625) (end 82.439375 109.51875) (width 0.3) (layer "F.Cu") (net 5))
 (segment (start 80.645 44.60875) (end 82.4635 46.42725) (width 0.3) (layer "F.Cu") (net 5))
 (segment (start 82.4635 46.42725) (end 82.4635 109.494625) (width 0.3) (layer "F.Cu") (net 5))
 (segment (start 125.415765 29.45525) (end 122.1288 32.742215) (width 0.3) (layer "B.Cu") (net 23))
 (segment (start 126.2785 29.45525) (end 125.415765 29.45525) (width 0.3) (layer "B.Cu") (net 23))
 (segment (start 108.90634 36.350032) (end 108.90634 37.56878) (width 0.3) (layer "B.Cu") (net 23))
 (segment (start 128.905 26.82875) (end 126.2785 29.45525) (width 0.3) (layer "B.Cu") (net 23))
 (segment (start 122.1288 32.742215) (end 112.514157 32.742215) (width 0.3) (layer "B.Cu") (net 23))
 (segment (start 112.514157 32.742215) (end 108.90634 36.350032) (width 0.3) (layer "B.Cu") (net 23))
 (segment (start 106.40634 34.08741) (end 106.40734 34.08641) (width 0.3) (layer "B.Cu") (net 27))
 (segment (start 106.40634 37.56878) (end 106.40634 34.08741) (width 0.3) (layer "B.Cu") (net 27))
 (segment (start 113.665 26.82875) (end 106.40734 34.08641) (width 0.3) (layer "B.Cu") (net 27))
 (segment (start 103.90634 27.23009) (end 103.90634 37.56878) (width 0.3) (layer "B.Cu") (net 31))
 (segment (start 103.505 26.82875) (end 103.90634 27.23009) (width 0.3) (layer "B.Cu") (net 31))
 (segment (start 109.40634 41.24741) (end 106.045 44.60875) (width 0.25) (layer "B.Cu") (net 14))
 (segment (start 109.40634 37.56878) (end 109.40634 41.24741) (width 0.25) (layer "B.Cu") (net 14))
 (segment (start 102.90634 33.85009) (end 95.885 26.82875) (width 0.3) (layer "B.Cu") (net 34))
 (segment (start 102.90634 37.56878) (end 102.90634 33.85009) (width 0.3) (layer "B.Cu") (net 34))
 (segment (start 104.90634 40.66741) (end 100.965 44.60875) (width 0.25) (layer "B.Cu") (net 12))
 (segment (start 104.90634 37.56878) (end 104.90634 40.66741) (width 0.25) (layer "B.Cu") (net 12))
 (segment (start 114.45875 42.8625) (end 116.205 44.60875) (width 0.25) (layer "B.Cu") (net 18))
 (segment (start 110.90634 37.56878) (end 110.90634 40.659465) (width 0.25) (layer "B.Cu") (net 18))
 (segment (start 110.90634 40.659465) (end 113.109375 42.8625) (width 0.25) (layer "B.Cu") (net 18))
 (segment (start 113.109375 42.8625) (end 114.45875 42.8625) (width 0.25) (layer "B.Cu") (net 18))
 (segment (start 121.86503 37.56878) (end 128.905 44.60875) (width 0.25) (layer "B.Cu") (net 22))
 (segment (start 112.90634 37.56878) (end 121.86503 37.56878) (width 0.25) (layer "B.Cu") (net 22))
 (segment (start 112.40095 32.146902) (end 108.40634 36.141512) (width 0.3) (layer "B.Cu") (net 24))
 (segment (start 121.046848 32.146902) (end 112.40095 32.146902) (width 0.3) (layer "B.Cu") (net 24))
 (segment (start 126.365 26.82875) (end 121.046848 32.146902) (width 0.3) (layer "B.Cu") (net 24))
 (segment (start 108.40634 36.141512) (end 108.40634 37.56878) (width 0.3) (layer "B.Cu") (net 24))
 (segment (start 105.90634 29.50741) (end 108.585 26.82875) (width 0.3) (layer "B.Cu") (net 29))
 (segment (start 105.90634 37.56878) (end 105.90634 29.50741) (width 0.3) (layer "B.Cu") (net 29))
 (segment (start 111.40634 37.56878) (end 111.40634 39.96884) (width 0.25) (layer "B.Cu") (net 19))
 (segment (start 111.40634 39.96884) (end 113.704723 42.267223) (width 0.25) (layer "B.Cu") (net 19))
 (segment (start 116.244723 42.267223) (end 118.58625 44.60875) (width 0.25) (layer "B.Cu") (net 19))
 (segment (start 118.58625 44.60875) (end 118.745 44.60875) (width 0.25) (layer "B.Cu") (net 19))
 (segment (start 113.704723 42.267223) (end 116.244723 42.267223) (width 0.25) (layer "B.Cu") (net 19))
 (segment (start 120.610387 36.98875) (end 132.8 36.98875) (width 0.3) (layer "F.Cu") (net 2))
 (segment (start 118.745 26.82875) (end 118.745 35.123363) (width 0.3) (layer "F.Cu") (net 2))
 (segment (start 119.340417 35.71878) (end 120.610387 36.98875) (width 0.3) (layer "F.Cu") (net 2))
 (segment (start 118.745 35.123363) (end 119.340417 35.71878) (width 0.3) (layer "F.Cu") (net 2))
 (segment (start 126.20625 54.76875) (end 129.778125 58.340625) (width 0.3) (layer "B.Cu") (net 2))
 (segment (start 135.73125 41.671875) (end 135.73125 39.92) (width 0.3) (layer "B.Cu") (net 2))
 (segment (start 140.49375 56.340625) (end 142.065625 56.340625) (width 0.3) (layer "B.Cu") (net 2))
 (segment (start 142.065625 56.340625) (end 142.72175 56.99675) (width 0.3) (layer "B.Cu") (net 2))
 (segment (start 142.72175 56.99675) (end 142.72175 61.242962) (width 0.3) (layer "B.Cu") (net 2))
 (segment (start 135.73125 39.92) (end 132.8 36.98875) (width 0.3) (layer "B.Cu") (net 2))
 (segment (start 114.428848 31.144902) (end 111.985908 31.144902) (width 0.3) (layer "B.Cu") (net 2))
 (segment (start 140.49375 56.340625) (end 140.49375 52.3875) (width 0.3) (layer "B.Cu") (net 2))
 (segment (start 140.49375 52.3875) (end 138.112616 50.006366) (width 0.3) (layer "B.Cu") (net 2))
 (segment (start 138.112616 50.006366) (end 138.112616 44.053241) (width 0.3) (layer "B.Cu") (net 2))
 (segment (start 142.72175 61.242962) (end 140.360587 63.604125) (width 0.3) (layer "B.Cu") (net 2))
 (segment (start 122.19375 55.489625) (end 122.19375 56.490625) (width 0.3) (layer "B.Cu") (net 2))
 (segment (start 122.914625 54.76875) (end 122.19375 55.489625) (width 0.3) (layer "B.Cu") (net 2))
 (segment (start 118.745 26.82875) (end 114.428848 31.144902) (width 0.3) (layer "B.Cu") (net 2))
 (segment (start 111.985908 31.144902) (end 107.40634 35.72447) (width 0.3) (layer "B.Cu") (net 2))
 (segment (start 140.360587 63.604125) (end 125.75525 63.604125) (width 0.3) (layer "B.Cu") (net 2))
 (segment (start 125.75525 63.604125) (end 122.19375 60.042625) (width 0.3) (layer "B.Cu") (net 2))
 (segment (start 122.19375 60.042625) (end 122.19375 56.490625) (width 0.3) (layer "B.Cu") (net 2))
 (segment (start 126.20625 54.76875) (end 122.914625 54.76875) (width 0.3) (layer "B.Cu") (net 2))
 (segment (start 138.112616 44.053241) (end 135.73125 41.671875) (width 0.3) (layer "B.Cu") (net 2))
 (segment (start 107.40634 35.72447) (end 107.40634 37.56878) (width 0.3) (layer "B.Cu") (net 2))
 (segment (start 129.778125 58.340625) (end 130.509375 58.340625) (width 0.3) (layer "B.Cu") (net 2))
 (segment (start 122.747913 40.991663) (end 126.365 44.60875) (width 0.25) (layer "B.Cu") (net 21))
 (segment (start 112.40634 39.69322) (end 113.704783 40.991663) (width 0.25) (layer "B.Cu") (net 21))
 (segment (start 112.40634 37.56878) (end 112.40634 39.69322) (width 0.25) (layer "B.Cu") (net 21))
 (segment (start 113.704783 40.991663) (end 122.747913 40.991663) (width 0.25) (layer "B.Cu") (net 21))
 (segment (start 103.160495 39.766625) (end 104.40634 38.52078) (width 0.25) (layer "B.Cu") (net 10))
 (segment (start 95.885 44.60875) (end 100.727125 39.766625) (width 0.25) (layer "B.Cu") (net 10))
 (segment (start 104.40634 38.52078) (end 104.40634 37.56878) (width 0.25) (layer "B.Cu") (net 10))
 (segment (start 100.727125 39.766625) (end 103.160495 39.766625) (width 0.25) (layer "B.Cu") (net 10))
 (segment (start 132.8 39.52875) (end 133.961 38.36775) (width 0.3) (layer "F.Cu") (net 1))
 (segment (start 133.961 36.507848) (end 133.280902 35.82775) (width 0.3) (layer "F.Cu") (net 1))
 (segment (start 133.280902 35.82775) (end 132.268375 35.82775) (width 0.3) (layer "F.Cu") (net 1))
 (segment (start 132.268375 35.82775) (end 129.778125 33.3375) (width 0.3) (layer "F.Cu") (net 1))
 (segment (start 131.887125 40.441625) (end 132.8 39.52875) (width 0.3) (layer "F.Cu") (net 1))
 (segment (start 129.778125 33.3375) (end 125.015625 33.3375) (width 0.3) (layer "F.Cu") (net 1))
 (segment (start 119.340417 39.290625) (end 120.491417 40.441625) (width 0.3) (layer "F.Cu") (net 1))
 (segment (start 125.015625 33.3375) (end 121.285 29.606875) (width 0.3) (layer "F.Cu") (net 1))
 (segment (start 120.491417 40.441625) (end 131.887125 40.441625) (width 0.3) (layer "F.Cu") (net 1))
 (segment (start 133.961 38.36775) (end 133.961 36.507848) (width 0.3) (layer "F.Cu") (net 1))
 (segment (start 121.285 29.606875) (end 121.285 26.82875) (width 0.3) (layer "F.Cu") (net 1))
 (segment (start 116.467848 31.645902) (end 112.193429 31.645902) (width 0.3) (layer "B.Cu") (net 1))
 (segment (start 142.22075 61.035442) (end 140.153067 63.103125) (width 0.3) (layer "B.Cu") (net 1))
 (segment (start 140.49375 57.340625) (end 141.220692 57.340625) (width 0.3) (layer "B.Cu") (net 1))
 (segment (start 112.193429 31.645902) (end 107.90634 35.932991) (width 0.3) (layer "B.Cu") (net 1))
 (segment (start 138.16975 54.089625) (end 138.16975 55.991625) (width 0.3) (layer "B.Cu") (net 1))
 (segment (start 141.220692 57.340625) (end 142.22075 58.340683) (width 0.3) (layer "B.Cu") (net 1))
 (segment (start 138.16975 55.991625) (end 139.51875 57.340625) (width 0.3) (layer "B.Cu") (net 1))
 (segment (start 122.69375 56.490625) (end 126.278125 56.490625) (width 0.3) (layer "B.Cu") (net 1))
 (segment (start 121.285 26.82875) (end 116.467848 31.645902) (width 0.3) (layer "B.Cu") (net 1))
 (segment (start 107.90634 35.932991) (end 107.90634 37.56878) (width 0.3) (layer "B.Cu") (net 1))
 (segment (start 135.742738 45.255238) (end 135.742738 51.662613) (width 0.3) (layer "B.Cu") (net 1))
 (segment (start 130.509375 60.721875) (end 132.890625 63.103125) (width 0.3) (layer "B.Cu") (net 1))
 (segment (start 142.22075 58.340683) (end 142.22075 61.035442) (width 0.3) (layer "B.Cu") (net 1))
 (segment (start 126.278125 56.490625) (end 130.509375 60.721875) (width 0.3) (layer "B.Cu") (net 1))
 (segment (start 135.742738 51.662613) (end 138.16975 54.089625) (width 0.3) (layer "B.Cu") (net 1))
 (segment (start 141.17075 57.340625) (end 140.49375 57.340625) (width 0.3) (layer "B.Cu") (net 1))
 (segment (start 132.8 39.52875) (end 132.8 42.3125) (width 0.3) (layer "B.Cu") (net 1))
 (segment (start 132.8 42.3125) (end 135.742738 45.255238) (width 0.3) (layer "B.Cu") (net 1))
 (segment (start 132.890625 63.103125) (end 140.153067 63.103125) (width 0.3) (layer "B.Cu") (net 1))
 (segment (start 139.51875 57.340625) (end 140.49375 57.340625) (width 0.3) (layer "B.Cu") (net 1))
 (segment (start 103.40634 37.56878) (end 103.40634 29.27009) (width 0.3) (layer "B.Cu") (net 32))
 (segment (start 103.40634 29.27009) (end 100.965 26.82875) (width 0.3) (layer "B.Cu") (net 32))
 (segment (start 103.505 44.60875) (end 105.40634 42.70741) (width 0.25) (layer "B.Cu") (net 13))
 (segment (start 105.40634 42.70741) (end 105.40634 37.56878) (width 0.25) (layer "B.Cu") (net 13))
 (segment (start 116.205 26.82875) (end 115.59354 26.82875) (width 0.3) (layer "B.Cu") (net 26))
 (segment (start 106.90634 35.51595) (end 106.90634 37.56878) (width 0.3) (layer "B.Cu") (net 26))
 (segment (start 115.59354 26.82875) (end 106.90634 35.51595) (width 0.3) (layer "B.Cu") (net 26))
 (segment (start 111.90634 39.83103) (end 113.726002 41.650692) (width 0.25) (layer "B.Cu") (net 20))
 (segment (start 113.726002 41.650692) (end 118.326942 41.650692) (width 0.25) (layer "B.Cu") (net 20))
 (segment (start 111.90634 37.56878) (end 111.90634 39.83103) (width 0.25) (layer "B.Cu") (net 20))
 (segment (start 118.326942 41.650692) (end 121.285 44.60875) (width 0.25) (layer "B.Cu") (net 20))
 (segment (start 92.474917 25.158833) (end 90.805 26.82875) (width 0.5) (layer "F.Cu") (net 3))
 (segment (start 132.8 34.44875) (end 134.061 33.18775) (width 0.5) (layer "F.Cu") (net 3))
 (segment (start 131.124547 25.158833) (end 92.474917 25.158833) (width 0.5) (layer "F.Cu") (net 3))
 (segment (start 134.061 33.18775) (end 134.061 28.095286) (width 0.5) (layer "F.Cu") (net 3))
 (segment (start 134.061 28.095286) (end 131.124547 25.158833) (width 0.5) (layer "F.Cu") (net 3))
 (segment (start 130.96875 36.28) (end 130.96875 43.393528) (width 0.5) (layer "B.Cu") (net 3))
 (segment (start 135.141738 56.530917) (end 136.951446 58.340625) (width 0.5) (layer "B.Cu") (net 3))
 (segment (start 141.61975 60.7865) (end 140.714625 61.691625) (width 0.5) (layer "B.Cu") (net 3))
 (segment (start 92.006 28.02975) (end 95.91931 28.02975) (width 0.3) (layer "B.Cu") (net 3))
 (segment (start 130.96875 36.28) (end 131.52997 35.71878) (width 0.5) (layer "B.Cu") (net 3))
 (segment (start 129.500417 35.71878) (end 131.52997 35.71878) (width 0.5) (layer "B.Cu") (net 3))
 (segment (start 132.159375 54.76875) (end 132.159375 58.340625) (width 0.3) (layer "B.Cu") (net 3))
 (segment (start 141.61975 58.589625) (end 141.61975 60.7865) (width 0.5) (layer "B.Cu") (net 3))
 (segment (start 129.778125 52.3875) (end 132.159375 54.76875) (width 0.3) (layer "B.Cu") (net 3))
 (segment (start 95.91931 28.02975) (end 102.40634 34.51678) (width 0.3) (layer "B.Cu") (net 3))
 (segment (start 133.129074 61.691625) (end 132.159375 60.721926) (width 0.5) (layer "B.Cu") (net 3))
 (segment (start 131.52997 35.71878) (end 132.8 34.44875) (width 0.5) (layer "B.Cu") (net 3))
 (segment (start 121.69375 54.51875) (end 123.825 52.3875) (width 0.3) (layer "B.Cu") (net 3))
 (segment (start 129.500417 35.71878) (end 129.500417 39.290625) (width 0.5) (layer "B.Cu") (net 3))
 (segment (start 121.69375 56.490625) (end 121.69375 54.51875) (width 0.3) (layer "B.Cu") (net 3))
 (segment (start 102.40634 34.51678) (end 102.40634 37.56878) (width 0.3) (layer "B.Cu") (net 3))
 (segment (start 130.96875 43.393528) (end 135.141738 47.566516) (width 0.5) (layer "B.Cu") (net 3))
 (segment (start 140.49375 58.340625) (end 141.37075 58.340625) (width 0.5) (layer "B.Cu") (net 3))
 (segment (start 132.159375 57.745422) (end 132.159375 58.340625) (width 0.3) (layer "B.Cu") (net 3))
 (segment (start 136.951446 58.340625) (end 140.49375 58.340625) (width 0.5) (layer "B.Cu") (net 3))
 (segment (start 135.141738 47.566516) (end 135.141738 56.530917) (width 0.5) (layer "B.Cu") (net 3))
 (segment (start 132.159375 60.721926) (end 132.159375 58.211926) (width 0.5) (layer "B.Cu") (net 3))
 (segment (start 123.825 52.3875) (end 129.778125 52.3875) (width 0.3) (layer "B.Cu") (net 3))
 (segment (start 133.129074 61.691625) (end 140.714625 61.691625) (width 0.5) (layer "B.Cu") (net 3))
 (segment (start 141.37075 58.340625) (end 141.61975 58.589625) (width 0.5) (layer "B.Cu") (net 3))
 (segment (start 90.805 26.82875) (end 92.006 28.02975) (width 0.3) (layer "B.Cu") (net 3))
 (segment (start 110.40634 41.35009) (end 113.665 44.60875) (width 0.25) (layer "B.Cu") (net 17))
 (segment (start 110.40634 37.56878) (end 110.40634 41.35009) (width 0.25) (layer "B.Cu") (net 17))
 (segment (start 109.90634 37.56878) (end 109.90634 43.28741) (width 0.25) (layer "B.Cu") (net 15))
 (segment (start 109.90634 43.28741) (end 108.585 44.60875) (width 0.25) (layer "B.Cu") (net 15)))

